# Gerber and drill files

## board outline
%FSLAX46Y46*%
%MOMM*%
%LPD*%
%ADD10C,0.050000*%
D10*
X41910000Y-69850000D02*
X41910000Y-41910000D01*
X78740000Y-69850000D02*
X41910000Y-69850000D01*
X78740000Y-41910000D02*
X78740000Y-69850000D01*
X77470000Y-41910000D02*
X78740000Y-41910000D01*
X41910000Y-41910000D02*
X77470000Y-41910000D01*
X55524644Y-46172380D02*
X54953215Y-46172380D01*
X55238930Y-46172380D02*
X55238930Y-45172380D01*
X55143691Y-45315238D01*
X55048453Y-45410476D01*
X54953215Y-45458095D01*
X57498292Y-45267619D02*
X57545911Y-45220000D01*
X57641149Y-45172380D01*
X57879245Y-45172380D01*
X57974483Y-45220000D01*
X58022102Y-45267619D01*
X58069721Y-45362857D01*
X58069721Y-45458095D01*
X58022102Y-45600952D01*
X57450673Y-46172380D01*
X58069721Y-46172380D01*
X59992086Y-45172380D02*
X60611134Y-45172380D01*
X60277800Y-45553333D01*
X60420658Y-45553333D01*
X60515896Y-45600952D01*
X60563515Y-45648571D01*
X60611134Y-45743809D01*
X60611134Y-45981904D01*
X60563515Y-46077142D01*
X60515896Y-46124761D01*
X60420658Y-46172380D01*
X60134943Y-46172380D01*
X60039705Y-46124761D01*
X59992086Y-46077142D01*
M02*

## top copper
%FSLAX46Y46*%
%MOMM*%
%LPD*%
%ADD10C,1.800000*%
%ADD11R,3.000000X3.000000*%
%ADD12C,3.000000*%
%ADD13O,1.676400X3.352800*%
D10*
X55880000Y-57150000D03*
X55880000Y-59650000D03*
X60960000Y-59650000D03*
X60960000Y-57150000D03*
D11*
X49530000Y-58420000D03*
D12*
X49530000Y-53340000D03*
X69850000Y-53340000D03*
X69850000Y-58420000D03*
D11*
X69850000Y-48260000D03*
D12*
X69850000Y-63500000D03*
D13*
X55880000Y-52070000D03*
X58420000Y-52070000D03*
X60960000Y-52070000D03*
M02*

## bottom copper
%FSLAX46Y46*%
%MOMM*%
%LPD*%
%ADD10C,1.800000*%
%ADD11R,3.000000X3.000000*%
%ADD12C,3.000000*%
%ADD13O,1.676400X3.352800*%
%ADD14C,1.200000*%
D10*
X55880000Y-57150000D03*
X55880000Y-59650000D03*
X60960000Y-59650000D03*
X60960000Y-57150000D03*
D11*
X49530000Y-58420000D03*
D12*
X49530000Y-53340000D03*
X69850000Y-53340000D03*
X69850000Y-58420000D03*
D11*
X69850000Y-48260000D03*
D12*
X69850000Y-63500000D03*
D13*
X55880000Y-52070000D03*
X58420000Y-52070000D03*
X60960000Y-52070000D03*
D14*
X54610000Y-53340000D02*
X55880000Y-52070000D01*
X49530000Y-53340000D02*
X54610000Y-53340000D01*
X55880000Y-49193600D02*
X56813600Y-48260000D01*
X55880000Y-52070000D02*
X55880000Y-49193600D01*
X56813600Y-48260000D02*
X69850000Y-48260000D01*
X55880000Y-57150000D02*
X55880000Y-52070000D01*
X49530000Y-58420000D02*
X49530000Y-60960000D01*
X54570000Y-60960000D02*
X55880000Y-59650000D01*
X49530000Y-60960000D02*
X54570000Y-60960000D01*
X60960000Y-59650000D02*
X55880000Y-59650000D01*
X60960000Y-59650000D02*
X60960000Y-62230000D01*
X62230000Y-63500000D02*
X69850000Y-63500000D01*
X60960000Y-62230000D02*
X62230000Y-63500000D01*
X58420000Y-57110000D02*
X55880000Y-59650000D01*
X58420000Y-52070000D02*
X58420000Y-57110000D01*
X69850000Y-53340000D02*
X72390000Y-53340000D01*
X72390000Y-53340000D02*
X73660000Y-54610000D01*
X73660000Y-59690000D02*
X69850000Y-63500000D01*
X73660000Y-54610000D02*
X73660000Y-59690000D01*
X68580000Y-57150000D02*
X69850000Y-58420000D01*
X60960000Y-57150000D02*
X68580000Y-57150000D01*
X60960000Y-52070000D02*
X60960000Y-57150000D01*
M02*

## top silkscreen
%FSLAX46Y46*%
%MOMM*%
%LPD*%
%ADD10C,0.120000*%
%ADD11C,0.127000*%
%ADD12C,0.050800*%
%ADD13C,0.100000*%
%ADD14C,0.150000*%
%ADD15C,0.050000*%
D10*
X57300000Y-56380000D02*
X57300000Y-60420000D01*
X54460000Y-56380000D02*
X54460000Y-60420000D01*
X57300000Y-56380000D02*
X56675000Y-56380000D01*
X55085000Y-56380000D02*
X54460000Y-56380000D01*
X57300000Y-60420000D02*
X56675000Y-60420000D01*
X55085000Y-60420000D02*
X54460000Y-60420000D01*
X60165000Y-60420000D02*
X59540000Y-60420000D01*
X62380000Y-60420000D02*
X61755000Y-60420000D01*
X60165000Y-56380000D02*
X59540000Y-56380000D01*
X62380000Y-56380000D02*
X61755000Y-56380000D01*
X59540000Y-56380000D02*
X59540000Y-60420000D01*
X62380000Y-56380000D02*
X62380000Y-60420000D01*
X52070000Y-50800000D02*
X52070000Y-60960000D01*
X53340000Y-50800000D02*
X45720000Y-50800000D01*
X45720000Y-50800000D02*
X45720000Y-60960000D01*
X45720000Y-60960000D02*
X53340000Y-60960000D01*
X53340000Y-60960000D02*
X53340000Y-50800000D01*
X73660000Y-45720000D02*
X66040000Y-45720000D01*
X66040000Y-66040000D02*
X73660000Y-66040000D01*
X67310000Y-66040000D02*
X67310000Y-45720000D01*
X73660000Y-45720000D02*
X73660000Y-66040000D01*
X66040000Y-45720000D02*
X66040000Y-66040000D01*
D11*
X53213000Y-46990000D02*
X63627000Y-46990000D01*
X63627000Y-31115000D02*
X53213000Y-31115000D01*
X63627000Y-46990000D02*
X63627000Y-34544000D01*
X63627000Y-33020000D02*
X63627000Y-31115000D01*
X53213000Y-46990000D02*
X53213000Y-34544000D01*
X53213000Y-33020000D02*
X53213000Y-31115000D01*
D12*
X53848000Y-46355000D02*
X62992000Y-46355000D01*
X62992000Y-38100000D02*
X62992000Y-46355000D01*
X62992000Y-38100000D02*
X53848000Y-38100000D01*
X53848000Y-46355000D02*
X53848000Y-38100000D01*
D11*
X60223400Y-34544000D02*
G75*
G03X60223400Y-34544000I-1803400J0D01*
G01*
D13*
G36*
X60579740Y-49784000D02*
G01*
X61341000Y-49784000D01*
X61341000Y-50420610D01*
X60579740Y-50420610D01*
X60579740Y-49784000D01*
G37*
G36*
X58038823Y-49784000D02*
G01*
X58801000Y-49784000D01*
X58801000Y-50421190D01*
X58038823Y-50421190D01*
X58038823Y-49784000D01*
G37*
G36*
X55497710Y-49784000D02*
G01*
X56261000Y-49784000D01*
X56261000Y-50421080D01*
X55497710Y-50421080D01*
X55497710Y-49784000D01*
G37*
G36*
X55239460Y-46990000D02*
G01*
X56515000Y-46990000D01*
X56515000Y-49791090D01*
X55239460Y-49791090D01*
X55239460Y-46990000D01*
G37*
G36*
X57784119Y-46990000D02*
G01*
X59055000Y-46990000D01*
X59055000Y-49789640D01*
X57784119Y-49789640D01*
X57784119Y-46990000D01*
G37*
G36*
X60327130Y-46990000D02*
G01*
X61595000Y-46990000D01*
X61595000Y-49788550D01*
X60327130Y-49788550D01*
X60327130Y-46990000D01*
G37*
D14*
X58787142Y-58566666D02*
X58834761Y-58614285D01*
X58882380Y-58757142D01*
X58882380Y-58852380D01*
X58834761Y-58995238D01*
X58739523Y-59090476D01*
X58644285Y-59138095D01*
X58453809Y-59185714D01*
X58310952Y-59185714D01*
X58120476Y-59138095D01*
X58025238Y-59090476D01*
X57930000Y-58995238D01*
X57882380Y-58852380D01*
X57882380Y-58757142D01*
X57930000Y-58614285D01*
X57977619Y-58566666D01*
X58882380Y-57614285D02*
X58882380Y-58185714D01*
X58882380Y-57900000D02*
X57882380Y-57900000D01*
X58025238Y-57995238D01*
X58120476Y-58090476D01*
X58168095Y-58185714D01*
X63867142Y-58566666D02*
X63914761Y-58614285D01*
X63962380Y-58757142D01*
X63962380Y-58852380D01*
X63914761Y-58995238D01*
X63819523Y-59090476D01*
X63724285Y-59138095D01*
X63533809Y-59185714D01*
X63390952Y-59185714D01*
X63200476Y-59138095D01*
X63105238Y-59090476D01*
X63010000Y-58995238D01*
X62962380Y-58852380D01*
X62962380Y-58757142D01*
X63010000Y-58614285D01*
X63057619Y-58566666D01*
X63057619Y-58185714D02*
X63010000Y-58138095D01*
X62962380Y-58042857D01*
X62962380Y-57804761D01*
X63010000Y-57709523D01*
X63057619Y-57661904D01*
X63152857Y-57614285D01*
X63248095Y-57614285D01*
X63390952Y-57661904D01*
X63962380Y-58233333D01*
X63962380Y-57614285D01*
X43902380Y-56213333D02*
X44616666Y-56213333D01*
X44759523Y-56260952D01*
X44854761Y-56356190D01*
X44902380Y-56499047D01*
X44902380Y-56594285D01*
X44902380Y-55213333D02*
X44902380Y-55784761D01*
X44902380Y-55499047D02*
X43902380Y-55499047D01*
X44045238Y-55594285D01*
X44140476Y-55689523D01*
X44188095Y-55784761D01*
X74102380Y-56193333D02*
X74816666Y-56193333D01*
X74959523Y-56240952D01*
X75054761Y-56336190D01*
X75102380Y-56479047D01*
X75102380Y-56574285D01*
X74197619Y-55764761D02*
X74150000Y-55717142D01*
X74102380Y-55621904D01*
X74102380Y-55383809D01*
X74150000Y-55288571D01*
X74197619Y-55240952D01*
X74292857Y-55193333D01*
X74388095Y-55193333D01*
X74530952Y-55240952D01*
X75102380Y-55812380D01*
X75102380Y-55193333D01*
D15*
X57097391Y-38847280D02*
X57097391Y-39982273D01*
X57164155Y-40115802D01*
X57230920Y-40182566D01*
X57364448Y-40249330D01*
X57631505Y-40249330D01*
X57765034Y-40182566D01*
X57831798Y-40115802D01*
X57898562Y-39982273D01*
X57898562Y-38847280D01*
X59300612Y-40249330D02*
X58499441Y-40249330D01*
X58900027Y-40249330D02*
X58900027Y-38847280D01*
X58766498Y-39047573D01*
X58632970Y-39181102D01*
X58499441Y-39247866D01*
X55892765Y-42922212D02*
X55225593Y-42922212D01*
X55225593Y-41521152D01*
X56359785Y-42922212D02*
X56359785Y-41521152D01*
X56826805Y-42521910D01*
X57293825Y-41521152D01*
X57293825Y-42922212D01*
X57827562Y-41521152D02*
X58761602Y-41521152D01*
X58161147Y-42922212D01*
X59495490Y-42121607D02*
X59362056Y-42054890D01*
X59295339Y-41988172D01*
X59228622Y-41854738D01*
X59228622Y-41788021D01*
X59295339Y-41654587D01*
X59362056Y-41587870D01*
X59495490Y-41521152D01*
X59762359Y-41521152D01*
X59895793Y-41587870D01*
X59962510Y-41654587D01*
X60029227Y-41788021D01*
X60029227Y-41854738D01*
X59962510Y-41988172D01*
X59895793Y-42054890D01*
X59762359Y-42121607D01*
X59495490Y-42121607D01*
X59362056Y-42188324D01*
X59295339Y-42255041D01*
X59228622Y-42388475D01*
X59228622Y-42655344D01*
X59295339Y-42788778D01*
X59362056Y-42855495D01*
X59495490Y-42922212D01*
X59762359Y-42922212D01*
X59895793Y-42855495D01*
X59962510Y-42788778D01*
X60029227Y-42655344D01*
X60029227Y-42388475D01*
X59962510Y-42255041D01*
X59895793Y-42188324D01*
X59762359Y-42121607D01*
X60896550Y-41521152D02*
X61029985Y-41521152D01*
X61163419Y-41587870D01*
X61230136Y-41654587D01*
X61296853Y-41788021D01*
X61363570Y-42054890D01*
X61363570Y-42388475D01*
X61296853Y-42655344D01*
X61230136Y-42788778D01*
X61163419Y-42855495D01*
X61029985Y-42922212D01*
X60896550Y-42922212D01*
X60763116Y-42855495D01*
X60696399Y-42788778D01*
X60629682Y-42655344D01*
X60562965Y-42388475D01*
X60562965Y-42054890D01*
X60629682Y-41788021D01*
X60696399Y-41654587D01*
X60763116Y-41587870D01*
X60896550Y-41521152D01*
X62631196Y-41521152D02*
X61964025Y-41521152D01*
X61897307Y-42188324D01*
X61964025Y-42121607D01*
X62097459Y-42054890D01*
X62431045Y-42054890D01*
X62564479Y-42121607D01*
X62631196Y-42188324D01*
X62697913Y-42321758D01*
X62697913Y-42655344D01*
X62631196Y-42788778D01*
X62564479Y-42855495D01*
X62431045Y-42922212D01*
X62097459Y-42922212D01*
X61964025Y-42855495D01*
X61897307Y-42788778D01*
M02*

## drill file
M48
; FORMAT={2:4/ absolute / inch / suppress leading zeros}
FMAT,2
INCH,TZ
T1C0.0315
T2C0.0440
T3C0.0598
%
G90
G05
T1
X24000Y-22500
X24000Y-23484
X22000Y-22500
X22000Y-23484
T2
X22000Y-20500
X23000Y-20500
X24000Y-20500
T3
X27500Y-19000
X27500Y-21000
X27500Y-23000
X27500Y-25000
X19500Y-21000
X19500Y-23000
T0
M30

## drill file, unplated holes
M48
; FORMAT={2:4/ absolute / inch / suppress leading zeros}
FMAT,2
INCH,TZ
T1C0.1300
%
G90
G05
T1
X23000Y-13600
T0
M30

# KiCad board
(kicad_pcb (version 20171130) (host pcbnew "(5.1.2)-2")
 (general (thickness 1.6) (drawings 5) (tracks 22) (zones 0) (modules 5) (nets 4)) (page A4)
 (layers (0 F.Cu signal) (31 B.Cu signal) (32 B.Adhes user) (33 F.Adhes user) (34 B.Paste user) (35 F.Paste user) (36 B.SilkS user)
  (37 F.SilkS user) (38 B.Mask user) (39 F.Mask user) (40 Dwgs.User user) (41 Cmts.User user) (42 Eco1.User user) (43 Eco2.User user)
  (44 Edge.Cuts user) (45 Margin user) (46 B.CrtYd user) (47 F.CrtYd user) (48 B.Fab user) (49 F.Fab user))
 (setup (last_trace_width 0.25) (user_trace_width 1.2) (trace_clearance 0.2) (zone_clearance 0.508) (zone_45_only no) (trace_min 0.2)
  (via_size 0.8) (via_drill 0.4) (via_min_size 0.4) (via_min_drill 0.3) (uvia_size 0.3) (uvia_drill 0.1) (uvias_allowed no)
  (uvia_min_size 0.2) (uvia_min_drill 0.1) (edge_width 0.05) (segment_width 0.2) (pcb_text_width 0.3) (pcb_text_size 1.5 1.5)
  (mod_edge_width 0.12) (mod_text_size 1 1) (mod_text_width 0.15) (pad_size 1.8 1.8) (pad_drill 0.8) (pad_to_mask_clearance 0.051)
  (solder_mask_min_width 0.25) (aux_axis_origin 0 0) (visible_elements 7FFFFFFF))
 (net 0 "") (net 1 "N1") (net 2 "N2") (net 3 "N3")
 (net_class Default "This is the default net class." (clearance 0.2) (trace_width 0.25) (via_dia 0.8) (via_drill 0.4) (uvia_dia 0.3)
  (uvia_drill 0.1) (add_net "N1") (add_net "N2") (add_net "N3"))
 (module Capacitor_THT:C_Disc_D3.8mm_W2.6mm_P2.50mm (layer F.Cu) (at 55.88 57.15 270)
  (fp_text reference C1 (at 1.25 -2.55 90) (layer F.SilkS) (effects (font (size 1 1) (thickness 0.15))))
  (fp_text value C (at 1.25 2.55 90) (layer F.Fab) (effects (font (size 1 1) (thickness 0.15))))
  (fp_line (start -0.77 -1.42) (end 3.27 -1.42) (layer F.SilkS) (width 0.12))
  (fp_line (start -0.77 1.42) (end 3.27 1.42) (layer F.SilkS) (width 0.12))
  (fp_line (start -0.77 -1.42) (end -0.77 -0.795) (layer F.SilkS) (width 0.12))
  (fp_line (start -0.77 0.795) (end -0.77 1.42) (layer F.SilkS) (width 0.12))
  (fp_line (start 3.27 -1.42) (end 3.27 -0.795) (layer F.SilkS) (width 0.12))
  (fp_line (start 3.27 0.795) (end 3.27 1.42) (layer F.SilkS) (width 0.12))
  (pad 1 thru_hole circle (at 0 0 270) (size 1.8 1.8) (drill 0.8) (layers *.Cu *.Mask) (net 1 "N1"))
  (pad 2 thru_hole circle (at 2.5 0 270) (size 1.8 1.8) (drill 0.8) (layers *.Cu *.Mask) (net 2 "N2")))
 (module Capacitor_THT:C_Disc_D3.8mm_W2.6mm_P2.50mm (layer F.Cu) (at 60.96 57.15 270)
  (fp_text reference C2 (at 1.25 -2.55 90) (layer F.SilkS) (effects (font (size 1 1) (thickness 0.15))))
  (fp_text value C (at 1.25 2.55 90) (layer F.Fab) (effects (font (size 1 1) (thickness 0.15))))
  (fp_line (start 3.27 0.795) (end 3.27 1.42) (layer F.SilkS) (width 0.12))
  (fp_line (start 3.27 -1.42) (end 3.27 -0.795) (layer F.SilkS) (width 0.12))
  (fp_line (start -0.77 0.795) (end -0.77 1.42) (layer F.SilkS) (width 0.12))
  (fp_line (start -0.77 -1.42) (end -0.77 -0.795) (layer F.SilkS) (width 0.12))
  (fp_line (start -0.77 1.42) (end 3.27 1.42) (layer F.SilkS) (width 0.12))
  (fp_line (start -0.77 -1.42) (end 3.27 -1.42) (layer F.SilkS) (width 0.12))
  (pad 2 thru_hole circle (at 2.5 0 270) (size 1.8 1.8) (drill 0.8) (layers *.Cu *.Mask) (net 2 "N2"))
  (pad 1 thru_hole circle (at 0 0 270) (size 1.8 1.8) (drill 0.8) (layers *.Cu *.Mask) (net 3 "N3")))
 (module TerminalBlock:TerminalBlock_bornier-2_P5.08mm (layer F.Cu) (at 49.53 58.42 90)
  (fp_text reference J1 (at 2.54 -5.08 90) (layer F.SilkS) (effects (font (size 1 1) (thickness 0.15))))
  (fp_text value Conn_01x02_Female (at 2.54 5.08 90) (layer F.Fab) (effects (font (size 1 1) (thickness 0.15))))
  (fp_line (start 7.62 2.54) (end -2.54 2.54) (layer F.SilkS) (width 0.12))
  (fp_line (start 7.62 3.81) (end 7.62 -3.81) (layer F.SilkS) (width 0.12))
  (fp_line (start 7.62 -3.81) (end -2.54 -3.81) (layer F.SilkS) (width 0.12))
  (fp_line (start -2.54 -3.81) (end -2.54 3.81) (layer F.SilkS) (width 0.12))
  (fp_line (start -2.54 3.81) (end 7.62 3.81) (layer F.SilkS) (width 0.12))
  (pad 1 thru_hole rect (at 0 0 90) (size 3 3) (drill 1.52) (layers *.Cu *.Mask) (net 2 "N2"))
  (pad 2 thru_hole circle (at 5.08 0 90) (size 3 3) (drill 1.52) (layers *.Cu *.Mask) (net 1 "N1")))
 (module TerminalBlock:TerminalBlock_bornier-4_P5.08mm (layer F.Cu) (at 69.85 48.26 270)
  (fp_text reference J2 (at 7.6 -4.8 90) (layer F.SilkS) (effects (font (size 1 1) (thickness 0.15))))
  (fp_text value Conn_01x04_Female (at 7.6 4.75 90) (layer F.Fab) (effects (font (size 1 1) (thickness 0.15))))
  (fp_line (start -2.54 -3.81) (end -2.54 3.81) (layer F.SilkS) (width 0.12))
  (fp_line (start 17.78 3.81) (end 17.78 -3.81) (layer F.SilkS) (width 0.12))
  (fp_line (start 17.78 2.54) (end -2.54 2.54) (layer F.SilkS) (width 0.12))
  (fp_line (start -2.54 -3.81) (end 17.78 -3.81) (layer F.SilkS) (width 0.12))
  (fp_line (start -2.54 3.81) (end 17.78 3.81) (layer F.SilkS) (width 0.12))
  (pad 2 thru_hole circle (at 5.08 0 270) (size 3 3) (drill 1.52) (layers *.Cu *.Mask) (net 2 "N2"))
  (pad 3 thru_hole circle (at 10.16 0 270) (size 3 3) (drill 1.52) (layers *.Cu *.Mask) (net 3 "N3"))
  (pad 1 thru_hole rect (at 0 0 270) (size 3 3) (drill 1.52) (layers *.Cu *.Mask) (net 1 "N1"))
  (pad 4 thru_hole circle (at 15.24 0 270) (size 3 3) (drill 1.52) (layers *.Cu *.Mask) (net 2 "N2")))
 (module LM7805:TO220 (layer F.Cu) (at 58.42 45.72)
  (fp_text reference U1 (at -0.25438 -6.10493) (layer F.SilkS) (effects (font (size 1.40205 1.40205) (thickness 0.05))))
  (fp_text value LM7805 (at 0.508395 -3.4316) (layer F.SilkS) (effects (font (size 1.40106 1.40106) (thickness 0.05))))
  (fp_line (start -5.207 1.27) (end 5.207 1.27) (layer F.SilkS) (width 0.127))
  (fp_line (start 5.207 -14.605) (end -5.207 -14.605) (layer F.SilkS) (width 0.127))
  (fp_line (start 5.207 1.27) (end 5.207 -11.176) (layer F.SilkS) (width 0.127))
  (fp_line (start 5.207 -12.7) (end 5.207 -14.605) (layer F.SilkS) (width 0.127))
  (fp_line (start -5.207 1.27) (end -5.207 -11.176) (layer F.SilkS) (width 0.127))
  (fp_line (start -5.207 -12.7) (end -5.207 -14.605) (layer F.SilkS) (width 0.127))
  (fp_line (start -4.572 0.635) (end 4.572 0.635) (layer F.SilkS) (width 0.0508))
  (fp_line (start 4.572 -7.62) (end 4.572 0.635) (layer F.SilkS) (width 0.0508))
  (fp_line (start 4.572 -7.62) (end -4.572 -7.62) (layer F.SilkS) (width 0.0508))
  (fp_line (start -4.572 0.635) (end -4.572 -7.62) (layer F.SilkS) (width 0.0508))
  (fp_circle (center 0 -11.176) (end 1.8034 -11.176) (layer F.SilkS) (width 0.127))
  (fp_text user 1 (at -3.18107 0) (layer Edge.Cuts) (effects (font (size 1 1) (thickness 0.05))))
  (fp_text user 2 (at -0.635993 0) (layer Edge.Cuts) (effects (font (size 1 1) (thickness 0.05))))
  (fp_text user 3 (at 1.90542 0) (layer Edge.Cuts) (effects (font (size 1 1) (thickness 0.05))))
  (fp_poly (pts (xy 2.15974 4.064) (xy 2.921 4.064) (xy 2.921 4.70061) (xy 2.15974 4.70061)) (layer F.SilkS) (width 0))
  (fp_poly (pts (xy -0.381177 4.064) (xy 0.381 4.064) (xy 0.381 4.70119) (xy -0.381177 4.70119)) (layer F.SilkS) (width 0))
  (fp_poly (pts (xy -2.92229 4.064) (xy -2.159 4.064) (xy -2.159 4.70108) (xy -2.92229 4.70108)) (layer F.SilkS) (width 0))
  (fp_poly (pts (xy -3.18054 1.27) (xy -1.905 1.27) (xy -1.905 4.07109) (xy -3.18054 4.07109)) (layer F.SilkS) (width 0))
  (fp_poly (pts (xy -0.635881 1.27) (xy 0.635 1.27) (xy 0.635 4.06964) (xy -0.635881 4.06964)) (layer F.SilkS) (width 0))
  (fp_poly (pts (xy 1.90713 1.27) (xy 3.175 1.27) (xy 3.175 4.06855) (xy 1.90713 4.06855)) (layer F.SilkS) (width 0))
  (pad 1 thru_hole oval (at -2.54 6.35 90) (size 3.3528 1.6764) (drill 1.1176) (layers *.Cu *.Mask) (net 1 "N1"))
  (pad 2 thru_hole oval (at 0 6.35 90) (size 3.3528 1.6764) (drill 1.1176) (layers *.Cu *.Mask) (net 2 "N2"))
  (pad 3 thru_hole oval (at 2.54 6.35 90) (size 3.3528 1.6764) (drill 1.1176) (layers *.Cu *.Mask) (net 3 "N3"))
  (pad Hole np_thru_hole circle (at 0 -11.176) (size 3.302 3.302) (drill 3.302) (layers *.Cu *.Mask F.SilkS)))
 (gr_line (start 41.91 69.85) (end 41.91 41.91) (layer Edge.Cuts) (width 0.05))
 (gr_line (start 78.74 69.85) (end 41.91 69.85) (layer Edge.Cuts) (width 0.05))
 (gr_line (start 78.74 41.91) (end 78.74 69.85) (layer Edge.Cuts) (width 0.05))
 (gr_line (start 77.47 41.91) (end 78.74 41.91) (layer Edge.Cuts) (width 0.05))
 (gr_line (start 41.91 41.91) (end 77.47 41.91) (layer Edge.Cuts) (width 0.05))
 (segment (start 54.61 53.34) (end 55.88 52.07) (width 1.2) (layer B.Cu) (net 1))
 (segment (start 49.53 53.34) (end 54.61 53.34) (width 1.2) (layer B.Cu) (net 1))
 (segment (start 55.88 49.1936) (end 56.8136 48.26) (width 1.2) (layer B.Cu) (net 1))
 (segment (start 55.88 52.07) (end 55.88 49.1936) (width 1.2) (layer B.Cu) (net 1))
 (segment (start 56.8136 48.26) (end 69.85 48.26) (width 1.2) (layer B.Cu) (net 1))
 (segment (start 55.88 57.15) (end 55.88 52.07) (width 1.2) (layer B.Cu) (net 1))
 (segment (start 49.53 58.42) (end 49.53 60.96) (width 1.2) (layer B.Cu) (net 2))
 (segment (start 54.57 60.96) (end 55.88 59.65) (width 1.2) (layer B.Cu) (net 2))
 (segment (start 49.53 60.96) (end 54.57 60.96) (width 1.2) (layer B.Cu) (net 2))
 (segment (start 60.96 59.65) (end 55.88 59.65) (width 1.2) (layer B.Cu) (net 2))
 (segment (start 60.96 59.65) (end 60.96 62.23) (width 1.2) (layer B.Cu) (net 2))
 (segment (start 62.23 63.5) (end 69.85 63.5) (width 1.2) (layer B.Cu) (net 2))
 (segment (start 60.96 62.23) (end 62.23 63.5) (width 1.2) (layer B.Cu) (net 2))
 (segment (start 58.42 57.11) (end 55.88 59.65) (width 1.2) (layer B.Cu) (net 2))
 (segment (start 58.42 52.07) (end 58.42 57.11) (width 1.2) (layer B.Cu) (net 2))
 (segment (start 69.85 53.34) (end 72.39 53.34) (width 1.2) (layer B.Cu) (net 2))
 (segment (start 72.39 53.34) (end 73.66 54.61) (width 1.2) (layer B.Cu) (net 2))
 (segment (start 73.66 59.69) (end 69.85 63.5) (width 1.2) (layer B.Cu) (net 2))
 (segment (start 73.66 54.61) (end 73.66 59.69) (width 1.2) (layer B.Cu) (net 2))
 (segment (start 68.58 57.15) (end 69.85 58.42) (width 1.2) (layer B.Cu) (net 3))
 (segment (start 60.96 57.15) (end 68.58 57.15) (width 1.2) (layer B.Cu) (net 3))
 (segment (start 60.96 52.07) (end 60.96 57.15) (width 1.2) (layer B.Cu) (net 3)))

